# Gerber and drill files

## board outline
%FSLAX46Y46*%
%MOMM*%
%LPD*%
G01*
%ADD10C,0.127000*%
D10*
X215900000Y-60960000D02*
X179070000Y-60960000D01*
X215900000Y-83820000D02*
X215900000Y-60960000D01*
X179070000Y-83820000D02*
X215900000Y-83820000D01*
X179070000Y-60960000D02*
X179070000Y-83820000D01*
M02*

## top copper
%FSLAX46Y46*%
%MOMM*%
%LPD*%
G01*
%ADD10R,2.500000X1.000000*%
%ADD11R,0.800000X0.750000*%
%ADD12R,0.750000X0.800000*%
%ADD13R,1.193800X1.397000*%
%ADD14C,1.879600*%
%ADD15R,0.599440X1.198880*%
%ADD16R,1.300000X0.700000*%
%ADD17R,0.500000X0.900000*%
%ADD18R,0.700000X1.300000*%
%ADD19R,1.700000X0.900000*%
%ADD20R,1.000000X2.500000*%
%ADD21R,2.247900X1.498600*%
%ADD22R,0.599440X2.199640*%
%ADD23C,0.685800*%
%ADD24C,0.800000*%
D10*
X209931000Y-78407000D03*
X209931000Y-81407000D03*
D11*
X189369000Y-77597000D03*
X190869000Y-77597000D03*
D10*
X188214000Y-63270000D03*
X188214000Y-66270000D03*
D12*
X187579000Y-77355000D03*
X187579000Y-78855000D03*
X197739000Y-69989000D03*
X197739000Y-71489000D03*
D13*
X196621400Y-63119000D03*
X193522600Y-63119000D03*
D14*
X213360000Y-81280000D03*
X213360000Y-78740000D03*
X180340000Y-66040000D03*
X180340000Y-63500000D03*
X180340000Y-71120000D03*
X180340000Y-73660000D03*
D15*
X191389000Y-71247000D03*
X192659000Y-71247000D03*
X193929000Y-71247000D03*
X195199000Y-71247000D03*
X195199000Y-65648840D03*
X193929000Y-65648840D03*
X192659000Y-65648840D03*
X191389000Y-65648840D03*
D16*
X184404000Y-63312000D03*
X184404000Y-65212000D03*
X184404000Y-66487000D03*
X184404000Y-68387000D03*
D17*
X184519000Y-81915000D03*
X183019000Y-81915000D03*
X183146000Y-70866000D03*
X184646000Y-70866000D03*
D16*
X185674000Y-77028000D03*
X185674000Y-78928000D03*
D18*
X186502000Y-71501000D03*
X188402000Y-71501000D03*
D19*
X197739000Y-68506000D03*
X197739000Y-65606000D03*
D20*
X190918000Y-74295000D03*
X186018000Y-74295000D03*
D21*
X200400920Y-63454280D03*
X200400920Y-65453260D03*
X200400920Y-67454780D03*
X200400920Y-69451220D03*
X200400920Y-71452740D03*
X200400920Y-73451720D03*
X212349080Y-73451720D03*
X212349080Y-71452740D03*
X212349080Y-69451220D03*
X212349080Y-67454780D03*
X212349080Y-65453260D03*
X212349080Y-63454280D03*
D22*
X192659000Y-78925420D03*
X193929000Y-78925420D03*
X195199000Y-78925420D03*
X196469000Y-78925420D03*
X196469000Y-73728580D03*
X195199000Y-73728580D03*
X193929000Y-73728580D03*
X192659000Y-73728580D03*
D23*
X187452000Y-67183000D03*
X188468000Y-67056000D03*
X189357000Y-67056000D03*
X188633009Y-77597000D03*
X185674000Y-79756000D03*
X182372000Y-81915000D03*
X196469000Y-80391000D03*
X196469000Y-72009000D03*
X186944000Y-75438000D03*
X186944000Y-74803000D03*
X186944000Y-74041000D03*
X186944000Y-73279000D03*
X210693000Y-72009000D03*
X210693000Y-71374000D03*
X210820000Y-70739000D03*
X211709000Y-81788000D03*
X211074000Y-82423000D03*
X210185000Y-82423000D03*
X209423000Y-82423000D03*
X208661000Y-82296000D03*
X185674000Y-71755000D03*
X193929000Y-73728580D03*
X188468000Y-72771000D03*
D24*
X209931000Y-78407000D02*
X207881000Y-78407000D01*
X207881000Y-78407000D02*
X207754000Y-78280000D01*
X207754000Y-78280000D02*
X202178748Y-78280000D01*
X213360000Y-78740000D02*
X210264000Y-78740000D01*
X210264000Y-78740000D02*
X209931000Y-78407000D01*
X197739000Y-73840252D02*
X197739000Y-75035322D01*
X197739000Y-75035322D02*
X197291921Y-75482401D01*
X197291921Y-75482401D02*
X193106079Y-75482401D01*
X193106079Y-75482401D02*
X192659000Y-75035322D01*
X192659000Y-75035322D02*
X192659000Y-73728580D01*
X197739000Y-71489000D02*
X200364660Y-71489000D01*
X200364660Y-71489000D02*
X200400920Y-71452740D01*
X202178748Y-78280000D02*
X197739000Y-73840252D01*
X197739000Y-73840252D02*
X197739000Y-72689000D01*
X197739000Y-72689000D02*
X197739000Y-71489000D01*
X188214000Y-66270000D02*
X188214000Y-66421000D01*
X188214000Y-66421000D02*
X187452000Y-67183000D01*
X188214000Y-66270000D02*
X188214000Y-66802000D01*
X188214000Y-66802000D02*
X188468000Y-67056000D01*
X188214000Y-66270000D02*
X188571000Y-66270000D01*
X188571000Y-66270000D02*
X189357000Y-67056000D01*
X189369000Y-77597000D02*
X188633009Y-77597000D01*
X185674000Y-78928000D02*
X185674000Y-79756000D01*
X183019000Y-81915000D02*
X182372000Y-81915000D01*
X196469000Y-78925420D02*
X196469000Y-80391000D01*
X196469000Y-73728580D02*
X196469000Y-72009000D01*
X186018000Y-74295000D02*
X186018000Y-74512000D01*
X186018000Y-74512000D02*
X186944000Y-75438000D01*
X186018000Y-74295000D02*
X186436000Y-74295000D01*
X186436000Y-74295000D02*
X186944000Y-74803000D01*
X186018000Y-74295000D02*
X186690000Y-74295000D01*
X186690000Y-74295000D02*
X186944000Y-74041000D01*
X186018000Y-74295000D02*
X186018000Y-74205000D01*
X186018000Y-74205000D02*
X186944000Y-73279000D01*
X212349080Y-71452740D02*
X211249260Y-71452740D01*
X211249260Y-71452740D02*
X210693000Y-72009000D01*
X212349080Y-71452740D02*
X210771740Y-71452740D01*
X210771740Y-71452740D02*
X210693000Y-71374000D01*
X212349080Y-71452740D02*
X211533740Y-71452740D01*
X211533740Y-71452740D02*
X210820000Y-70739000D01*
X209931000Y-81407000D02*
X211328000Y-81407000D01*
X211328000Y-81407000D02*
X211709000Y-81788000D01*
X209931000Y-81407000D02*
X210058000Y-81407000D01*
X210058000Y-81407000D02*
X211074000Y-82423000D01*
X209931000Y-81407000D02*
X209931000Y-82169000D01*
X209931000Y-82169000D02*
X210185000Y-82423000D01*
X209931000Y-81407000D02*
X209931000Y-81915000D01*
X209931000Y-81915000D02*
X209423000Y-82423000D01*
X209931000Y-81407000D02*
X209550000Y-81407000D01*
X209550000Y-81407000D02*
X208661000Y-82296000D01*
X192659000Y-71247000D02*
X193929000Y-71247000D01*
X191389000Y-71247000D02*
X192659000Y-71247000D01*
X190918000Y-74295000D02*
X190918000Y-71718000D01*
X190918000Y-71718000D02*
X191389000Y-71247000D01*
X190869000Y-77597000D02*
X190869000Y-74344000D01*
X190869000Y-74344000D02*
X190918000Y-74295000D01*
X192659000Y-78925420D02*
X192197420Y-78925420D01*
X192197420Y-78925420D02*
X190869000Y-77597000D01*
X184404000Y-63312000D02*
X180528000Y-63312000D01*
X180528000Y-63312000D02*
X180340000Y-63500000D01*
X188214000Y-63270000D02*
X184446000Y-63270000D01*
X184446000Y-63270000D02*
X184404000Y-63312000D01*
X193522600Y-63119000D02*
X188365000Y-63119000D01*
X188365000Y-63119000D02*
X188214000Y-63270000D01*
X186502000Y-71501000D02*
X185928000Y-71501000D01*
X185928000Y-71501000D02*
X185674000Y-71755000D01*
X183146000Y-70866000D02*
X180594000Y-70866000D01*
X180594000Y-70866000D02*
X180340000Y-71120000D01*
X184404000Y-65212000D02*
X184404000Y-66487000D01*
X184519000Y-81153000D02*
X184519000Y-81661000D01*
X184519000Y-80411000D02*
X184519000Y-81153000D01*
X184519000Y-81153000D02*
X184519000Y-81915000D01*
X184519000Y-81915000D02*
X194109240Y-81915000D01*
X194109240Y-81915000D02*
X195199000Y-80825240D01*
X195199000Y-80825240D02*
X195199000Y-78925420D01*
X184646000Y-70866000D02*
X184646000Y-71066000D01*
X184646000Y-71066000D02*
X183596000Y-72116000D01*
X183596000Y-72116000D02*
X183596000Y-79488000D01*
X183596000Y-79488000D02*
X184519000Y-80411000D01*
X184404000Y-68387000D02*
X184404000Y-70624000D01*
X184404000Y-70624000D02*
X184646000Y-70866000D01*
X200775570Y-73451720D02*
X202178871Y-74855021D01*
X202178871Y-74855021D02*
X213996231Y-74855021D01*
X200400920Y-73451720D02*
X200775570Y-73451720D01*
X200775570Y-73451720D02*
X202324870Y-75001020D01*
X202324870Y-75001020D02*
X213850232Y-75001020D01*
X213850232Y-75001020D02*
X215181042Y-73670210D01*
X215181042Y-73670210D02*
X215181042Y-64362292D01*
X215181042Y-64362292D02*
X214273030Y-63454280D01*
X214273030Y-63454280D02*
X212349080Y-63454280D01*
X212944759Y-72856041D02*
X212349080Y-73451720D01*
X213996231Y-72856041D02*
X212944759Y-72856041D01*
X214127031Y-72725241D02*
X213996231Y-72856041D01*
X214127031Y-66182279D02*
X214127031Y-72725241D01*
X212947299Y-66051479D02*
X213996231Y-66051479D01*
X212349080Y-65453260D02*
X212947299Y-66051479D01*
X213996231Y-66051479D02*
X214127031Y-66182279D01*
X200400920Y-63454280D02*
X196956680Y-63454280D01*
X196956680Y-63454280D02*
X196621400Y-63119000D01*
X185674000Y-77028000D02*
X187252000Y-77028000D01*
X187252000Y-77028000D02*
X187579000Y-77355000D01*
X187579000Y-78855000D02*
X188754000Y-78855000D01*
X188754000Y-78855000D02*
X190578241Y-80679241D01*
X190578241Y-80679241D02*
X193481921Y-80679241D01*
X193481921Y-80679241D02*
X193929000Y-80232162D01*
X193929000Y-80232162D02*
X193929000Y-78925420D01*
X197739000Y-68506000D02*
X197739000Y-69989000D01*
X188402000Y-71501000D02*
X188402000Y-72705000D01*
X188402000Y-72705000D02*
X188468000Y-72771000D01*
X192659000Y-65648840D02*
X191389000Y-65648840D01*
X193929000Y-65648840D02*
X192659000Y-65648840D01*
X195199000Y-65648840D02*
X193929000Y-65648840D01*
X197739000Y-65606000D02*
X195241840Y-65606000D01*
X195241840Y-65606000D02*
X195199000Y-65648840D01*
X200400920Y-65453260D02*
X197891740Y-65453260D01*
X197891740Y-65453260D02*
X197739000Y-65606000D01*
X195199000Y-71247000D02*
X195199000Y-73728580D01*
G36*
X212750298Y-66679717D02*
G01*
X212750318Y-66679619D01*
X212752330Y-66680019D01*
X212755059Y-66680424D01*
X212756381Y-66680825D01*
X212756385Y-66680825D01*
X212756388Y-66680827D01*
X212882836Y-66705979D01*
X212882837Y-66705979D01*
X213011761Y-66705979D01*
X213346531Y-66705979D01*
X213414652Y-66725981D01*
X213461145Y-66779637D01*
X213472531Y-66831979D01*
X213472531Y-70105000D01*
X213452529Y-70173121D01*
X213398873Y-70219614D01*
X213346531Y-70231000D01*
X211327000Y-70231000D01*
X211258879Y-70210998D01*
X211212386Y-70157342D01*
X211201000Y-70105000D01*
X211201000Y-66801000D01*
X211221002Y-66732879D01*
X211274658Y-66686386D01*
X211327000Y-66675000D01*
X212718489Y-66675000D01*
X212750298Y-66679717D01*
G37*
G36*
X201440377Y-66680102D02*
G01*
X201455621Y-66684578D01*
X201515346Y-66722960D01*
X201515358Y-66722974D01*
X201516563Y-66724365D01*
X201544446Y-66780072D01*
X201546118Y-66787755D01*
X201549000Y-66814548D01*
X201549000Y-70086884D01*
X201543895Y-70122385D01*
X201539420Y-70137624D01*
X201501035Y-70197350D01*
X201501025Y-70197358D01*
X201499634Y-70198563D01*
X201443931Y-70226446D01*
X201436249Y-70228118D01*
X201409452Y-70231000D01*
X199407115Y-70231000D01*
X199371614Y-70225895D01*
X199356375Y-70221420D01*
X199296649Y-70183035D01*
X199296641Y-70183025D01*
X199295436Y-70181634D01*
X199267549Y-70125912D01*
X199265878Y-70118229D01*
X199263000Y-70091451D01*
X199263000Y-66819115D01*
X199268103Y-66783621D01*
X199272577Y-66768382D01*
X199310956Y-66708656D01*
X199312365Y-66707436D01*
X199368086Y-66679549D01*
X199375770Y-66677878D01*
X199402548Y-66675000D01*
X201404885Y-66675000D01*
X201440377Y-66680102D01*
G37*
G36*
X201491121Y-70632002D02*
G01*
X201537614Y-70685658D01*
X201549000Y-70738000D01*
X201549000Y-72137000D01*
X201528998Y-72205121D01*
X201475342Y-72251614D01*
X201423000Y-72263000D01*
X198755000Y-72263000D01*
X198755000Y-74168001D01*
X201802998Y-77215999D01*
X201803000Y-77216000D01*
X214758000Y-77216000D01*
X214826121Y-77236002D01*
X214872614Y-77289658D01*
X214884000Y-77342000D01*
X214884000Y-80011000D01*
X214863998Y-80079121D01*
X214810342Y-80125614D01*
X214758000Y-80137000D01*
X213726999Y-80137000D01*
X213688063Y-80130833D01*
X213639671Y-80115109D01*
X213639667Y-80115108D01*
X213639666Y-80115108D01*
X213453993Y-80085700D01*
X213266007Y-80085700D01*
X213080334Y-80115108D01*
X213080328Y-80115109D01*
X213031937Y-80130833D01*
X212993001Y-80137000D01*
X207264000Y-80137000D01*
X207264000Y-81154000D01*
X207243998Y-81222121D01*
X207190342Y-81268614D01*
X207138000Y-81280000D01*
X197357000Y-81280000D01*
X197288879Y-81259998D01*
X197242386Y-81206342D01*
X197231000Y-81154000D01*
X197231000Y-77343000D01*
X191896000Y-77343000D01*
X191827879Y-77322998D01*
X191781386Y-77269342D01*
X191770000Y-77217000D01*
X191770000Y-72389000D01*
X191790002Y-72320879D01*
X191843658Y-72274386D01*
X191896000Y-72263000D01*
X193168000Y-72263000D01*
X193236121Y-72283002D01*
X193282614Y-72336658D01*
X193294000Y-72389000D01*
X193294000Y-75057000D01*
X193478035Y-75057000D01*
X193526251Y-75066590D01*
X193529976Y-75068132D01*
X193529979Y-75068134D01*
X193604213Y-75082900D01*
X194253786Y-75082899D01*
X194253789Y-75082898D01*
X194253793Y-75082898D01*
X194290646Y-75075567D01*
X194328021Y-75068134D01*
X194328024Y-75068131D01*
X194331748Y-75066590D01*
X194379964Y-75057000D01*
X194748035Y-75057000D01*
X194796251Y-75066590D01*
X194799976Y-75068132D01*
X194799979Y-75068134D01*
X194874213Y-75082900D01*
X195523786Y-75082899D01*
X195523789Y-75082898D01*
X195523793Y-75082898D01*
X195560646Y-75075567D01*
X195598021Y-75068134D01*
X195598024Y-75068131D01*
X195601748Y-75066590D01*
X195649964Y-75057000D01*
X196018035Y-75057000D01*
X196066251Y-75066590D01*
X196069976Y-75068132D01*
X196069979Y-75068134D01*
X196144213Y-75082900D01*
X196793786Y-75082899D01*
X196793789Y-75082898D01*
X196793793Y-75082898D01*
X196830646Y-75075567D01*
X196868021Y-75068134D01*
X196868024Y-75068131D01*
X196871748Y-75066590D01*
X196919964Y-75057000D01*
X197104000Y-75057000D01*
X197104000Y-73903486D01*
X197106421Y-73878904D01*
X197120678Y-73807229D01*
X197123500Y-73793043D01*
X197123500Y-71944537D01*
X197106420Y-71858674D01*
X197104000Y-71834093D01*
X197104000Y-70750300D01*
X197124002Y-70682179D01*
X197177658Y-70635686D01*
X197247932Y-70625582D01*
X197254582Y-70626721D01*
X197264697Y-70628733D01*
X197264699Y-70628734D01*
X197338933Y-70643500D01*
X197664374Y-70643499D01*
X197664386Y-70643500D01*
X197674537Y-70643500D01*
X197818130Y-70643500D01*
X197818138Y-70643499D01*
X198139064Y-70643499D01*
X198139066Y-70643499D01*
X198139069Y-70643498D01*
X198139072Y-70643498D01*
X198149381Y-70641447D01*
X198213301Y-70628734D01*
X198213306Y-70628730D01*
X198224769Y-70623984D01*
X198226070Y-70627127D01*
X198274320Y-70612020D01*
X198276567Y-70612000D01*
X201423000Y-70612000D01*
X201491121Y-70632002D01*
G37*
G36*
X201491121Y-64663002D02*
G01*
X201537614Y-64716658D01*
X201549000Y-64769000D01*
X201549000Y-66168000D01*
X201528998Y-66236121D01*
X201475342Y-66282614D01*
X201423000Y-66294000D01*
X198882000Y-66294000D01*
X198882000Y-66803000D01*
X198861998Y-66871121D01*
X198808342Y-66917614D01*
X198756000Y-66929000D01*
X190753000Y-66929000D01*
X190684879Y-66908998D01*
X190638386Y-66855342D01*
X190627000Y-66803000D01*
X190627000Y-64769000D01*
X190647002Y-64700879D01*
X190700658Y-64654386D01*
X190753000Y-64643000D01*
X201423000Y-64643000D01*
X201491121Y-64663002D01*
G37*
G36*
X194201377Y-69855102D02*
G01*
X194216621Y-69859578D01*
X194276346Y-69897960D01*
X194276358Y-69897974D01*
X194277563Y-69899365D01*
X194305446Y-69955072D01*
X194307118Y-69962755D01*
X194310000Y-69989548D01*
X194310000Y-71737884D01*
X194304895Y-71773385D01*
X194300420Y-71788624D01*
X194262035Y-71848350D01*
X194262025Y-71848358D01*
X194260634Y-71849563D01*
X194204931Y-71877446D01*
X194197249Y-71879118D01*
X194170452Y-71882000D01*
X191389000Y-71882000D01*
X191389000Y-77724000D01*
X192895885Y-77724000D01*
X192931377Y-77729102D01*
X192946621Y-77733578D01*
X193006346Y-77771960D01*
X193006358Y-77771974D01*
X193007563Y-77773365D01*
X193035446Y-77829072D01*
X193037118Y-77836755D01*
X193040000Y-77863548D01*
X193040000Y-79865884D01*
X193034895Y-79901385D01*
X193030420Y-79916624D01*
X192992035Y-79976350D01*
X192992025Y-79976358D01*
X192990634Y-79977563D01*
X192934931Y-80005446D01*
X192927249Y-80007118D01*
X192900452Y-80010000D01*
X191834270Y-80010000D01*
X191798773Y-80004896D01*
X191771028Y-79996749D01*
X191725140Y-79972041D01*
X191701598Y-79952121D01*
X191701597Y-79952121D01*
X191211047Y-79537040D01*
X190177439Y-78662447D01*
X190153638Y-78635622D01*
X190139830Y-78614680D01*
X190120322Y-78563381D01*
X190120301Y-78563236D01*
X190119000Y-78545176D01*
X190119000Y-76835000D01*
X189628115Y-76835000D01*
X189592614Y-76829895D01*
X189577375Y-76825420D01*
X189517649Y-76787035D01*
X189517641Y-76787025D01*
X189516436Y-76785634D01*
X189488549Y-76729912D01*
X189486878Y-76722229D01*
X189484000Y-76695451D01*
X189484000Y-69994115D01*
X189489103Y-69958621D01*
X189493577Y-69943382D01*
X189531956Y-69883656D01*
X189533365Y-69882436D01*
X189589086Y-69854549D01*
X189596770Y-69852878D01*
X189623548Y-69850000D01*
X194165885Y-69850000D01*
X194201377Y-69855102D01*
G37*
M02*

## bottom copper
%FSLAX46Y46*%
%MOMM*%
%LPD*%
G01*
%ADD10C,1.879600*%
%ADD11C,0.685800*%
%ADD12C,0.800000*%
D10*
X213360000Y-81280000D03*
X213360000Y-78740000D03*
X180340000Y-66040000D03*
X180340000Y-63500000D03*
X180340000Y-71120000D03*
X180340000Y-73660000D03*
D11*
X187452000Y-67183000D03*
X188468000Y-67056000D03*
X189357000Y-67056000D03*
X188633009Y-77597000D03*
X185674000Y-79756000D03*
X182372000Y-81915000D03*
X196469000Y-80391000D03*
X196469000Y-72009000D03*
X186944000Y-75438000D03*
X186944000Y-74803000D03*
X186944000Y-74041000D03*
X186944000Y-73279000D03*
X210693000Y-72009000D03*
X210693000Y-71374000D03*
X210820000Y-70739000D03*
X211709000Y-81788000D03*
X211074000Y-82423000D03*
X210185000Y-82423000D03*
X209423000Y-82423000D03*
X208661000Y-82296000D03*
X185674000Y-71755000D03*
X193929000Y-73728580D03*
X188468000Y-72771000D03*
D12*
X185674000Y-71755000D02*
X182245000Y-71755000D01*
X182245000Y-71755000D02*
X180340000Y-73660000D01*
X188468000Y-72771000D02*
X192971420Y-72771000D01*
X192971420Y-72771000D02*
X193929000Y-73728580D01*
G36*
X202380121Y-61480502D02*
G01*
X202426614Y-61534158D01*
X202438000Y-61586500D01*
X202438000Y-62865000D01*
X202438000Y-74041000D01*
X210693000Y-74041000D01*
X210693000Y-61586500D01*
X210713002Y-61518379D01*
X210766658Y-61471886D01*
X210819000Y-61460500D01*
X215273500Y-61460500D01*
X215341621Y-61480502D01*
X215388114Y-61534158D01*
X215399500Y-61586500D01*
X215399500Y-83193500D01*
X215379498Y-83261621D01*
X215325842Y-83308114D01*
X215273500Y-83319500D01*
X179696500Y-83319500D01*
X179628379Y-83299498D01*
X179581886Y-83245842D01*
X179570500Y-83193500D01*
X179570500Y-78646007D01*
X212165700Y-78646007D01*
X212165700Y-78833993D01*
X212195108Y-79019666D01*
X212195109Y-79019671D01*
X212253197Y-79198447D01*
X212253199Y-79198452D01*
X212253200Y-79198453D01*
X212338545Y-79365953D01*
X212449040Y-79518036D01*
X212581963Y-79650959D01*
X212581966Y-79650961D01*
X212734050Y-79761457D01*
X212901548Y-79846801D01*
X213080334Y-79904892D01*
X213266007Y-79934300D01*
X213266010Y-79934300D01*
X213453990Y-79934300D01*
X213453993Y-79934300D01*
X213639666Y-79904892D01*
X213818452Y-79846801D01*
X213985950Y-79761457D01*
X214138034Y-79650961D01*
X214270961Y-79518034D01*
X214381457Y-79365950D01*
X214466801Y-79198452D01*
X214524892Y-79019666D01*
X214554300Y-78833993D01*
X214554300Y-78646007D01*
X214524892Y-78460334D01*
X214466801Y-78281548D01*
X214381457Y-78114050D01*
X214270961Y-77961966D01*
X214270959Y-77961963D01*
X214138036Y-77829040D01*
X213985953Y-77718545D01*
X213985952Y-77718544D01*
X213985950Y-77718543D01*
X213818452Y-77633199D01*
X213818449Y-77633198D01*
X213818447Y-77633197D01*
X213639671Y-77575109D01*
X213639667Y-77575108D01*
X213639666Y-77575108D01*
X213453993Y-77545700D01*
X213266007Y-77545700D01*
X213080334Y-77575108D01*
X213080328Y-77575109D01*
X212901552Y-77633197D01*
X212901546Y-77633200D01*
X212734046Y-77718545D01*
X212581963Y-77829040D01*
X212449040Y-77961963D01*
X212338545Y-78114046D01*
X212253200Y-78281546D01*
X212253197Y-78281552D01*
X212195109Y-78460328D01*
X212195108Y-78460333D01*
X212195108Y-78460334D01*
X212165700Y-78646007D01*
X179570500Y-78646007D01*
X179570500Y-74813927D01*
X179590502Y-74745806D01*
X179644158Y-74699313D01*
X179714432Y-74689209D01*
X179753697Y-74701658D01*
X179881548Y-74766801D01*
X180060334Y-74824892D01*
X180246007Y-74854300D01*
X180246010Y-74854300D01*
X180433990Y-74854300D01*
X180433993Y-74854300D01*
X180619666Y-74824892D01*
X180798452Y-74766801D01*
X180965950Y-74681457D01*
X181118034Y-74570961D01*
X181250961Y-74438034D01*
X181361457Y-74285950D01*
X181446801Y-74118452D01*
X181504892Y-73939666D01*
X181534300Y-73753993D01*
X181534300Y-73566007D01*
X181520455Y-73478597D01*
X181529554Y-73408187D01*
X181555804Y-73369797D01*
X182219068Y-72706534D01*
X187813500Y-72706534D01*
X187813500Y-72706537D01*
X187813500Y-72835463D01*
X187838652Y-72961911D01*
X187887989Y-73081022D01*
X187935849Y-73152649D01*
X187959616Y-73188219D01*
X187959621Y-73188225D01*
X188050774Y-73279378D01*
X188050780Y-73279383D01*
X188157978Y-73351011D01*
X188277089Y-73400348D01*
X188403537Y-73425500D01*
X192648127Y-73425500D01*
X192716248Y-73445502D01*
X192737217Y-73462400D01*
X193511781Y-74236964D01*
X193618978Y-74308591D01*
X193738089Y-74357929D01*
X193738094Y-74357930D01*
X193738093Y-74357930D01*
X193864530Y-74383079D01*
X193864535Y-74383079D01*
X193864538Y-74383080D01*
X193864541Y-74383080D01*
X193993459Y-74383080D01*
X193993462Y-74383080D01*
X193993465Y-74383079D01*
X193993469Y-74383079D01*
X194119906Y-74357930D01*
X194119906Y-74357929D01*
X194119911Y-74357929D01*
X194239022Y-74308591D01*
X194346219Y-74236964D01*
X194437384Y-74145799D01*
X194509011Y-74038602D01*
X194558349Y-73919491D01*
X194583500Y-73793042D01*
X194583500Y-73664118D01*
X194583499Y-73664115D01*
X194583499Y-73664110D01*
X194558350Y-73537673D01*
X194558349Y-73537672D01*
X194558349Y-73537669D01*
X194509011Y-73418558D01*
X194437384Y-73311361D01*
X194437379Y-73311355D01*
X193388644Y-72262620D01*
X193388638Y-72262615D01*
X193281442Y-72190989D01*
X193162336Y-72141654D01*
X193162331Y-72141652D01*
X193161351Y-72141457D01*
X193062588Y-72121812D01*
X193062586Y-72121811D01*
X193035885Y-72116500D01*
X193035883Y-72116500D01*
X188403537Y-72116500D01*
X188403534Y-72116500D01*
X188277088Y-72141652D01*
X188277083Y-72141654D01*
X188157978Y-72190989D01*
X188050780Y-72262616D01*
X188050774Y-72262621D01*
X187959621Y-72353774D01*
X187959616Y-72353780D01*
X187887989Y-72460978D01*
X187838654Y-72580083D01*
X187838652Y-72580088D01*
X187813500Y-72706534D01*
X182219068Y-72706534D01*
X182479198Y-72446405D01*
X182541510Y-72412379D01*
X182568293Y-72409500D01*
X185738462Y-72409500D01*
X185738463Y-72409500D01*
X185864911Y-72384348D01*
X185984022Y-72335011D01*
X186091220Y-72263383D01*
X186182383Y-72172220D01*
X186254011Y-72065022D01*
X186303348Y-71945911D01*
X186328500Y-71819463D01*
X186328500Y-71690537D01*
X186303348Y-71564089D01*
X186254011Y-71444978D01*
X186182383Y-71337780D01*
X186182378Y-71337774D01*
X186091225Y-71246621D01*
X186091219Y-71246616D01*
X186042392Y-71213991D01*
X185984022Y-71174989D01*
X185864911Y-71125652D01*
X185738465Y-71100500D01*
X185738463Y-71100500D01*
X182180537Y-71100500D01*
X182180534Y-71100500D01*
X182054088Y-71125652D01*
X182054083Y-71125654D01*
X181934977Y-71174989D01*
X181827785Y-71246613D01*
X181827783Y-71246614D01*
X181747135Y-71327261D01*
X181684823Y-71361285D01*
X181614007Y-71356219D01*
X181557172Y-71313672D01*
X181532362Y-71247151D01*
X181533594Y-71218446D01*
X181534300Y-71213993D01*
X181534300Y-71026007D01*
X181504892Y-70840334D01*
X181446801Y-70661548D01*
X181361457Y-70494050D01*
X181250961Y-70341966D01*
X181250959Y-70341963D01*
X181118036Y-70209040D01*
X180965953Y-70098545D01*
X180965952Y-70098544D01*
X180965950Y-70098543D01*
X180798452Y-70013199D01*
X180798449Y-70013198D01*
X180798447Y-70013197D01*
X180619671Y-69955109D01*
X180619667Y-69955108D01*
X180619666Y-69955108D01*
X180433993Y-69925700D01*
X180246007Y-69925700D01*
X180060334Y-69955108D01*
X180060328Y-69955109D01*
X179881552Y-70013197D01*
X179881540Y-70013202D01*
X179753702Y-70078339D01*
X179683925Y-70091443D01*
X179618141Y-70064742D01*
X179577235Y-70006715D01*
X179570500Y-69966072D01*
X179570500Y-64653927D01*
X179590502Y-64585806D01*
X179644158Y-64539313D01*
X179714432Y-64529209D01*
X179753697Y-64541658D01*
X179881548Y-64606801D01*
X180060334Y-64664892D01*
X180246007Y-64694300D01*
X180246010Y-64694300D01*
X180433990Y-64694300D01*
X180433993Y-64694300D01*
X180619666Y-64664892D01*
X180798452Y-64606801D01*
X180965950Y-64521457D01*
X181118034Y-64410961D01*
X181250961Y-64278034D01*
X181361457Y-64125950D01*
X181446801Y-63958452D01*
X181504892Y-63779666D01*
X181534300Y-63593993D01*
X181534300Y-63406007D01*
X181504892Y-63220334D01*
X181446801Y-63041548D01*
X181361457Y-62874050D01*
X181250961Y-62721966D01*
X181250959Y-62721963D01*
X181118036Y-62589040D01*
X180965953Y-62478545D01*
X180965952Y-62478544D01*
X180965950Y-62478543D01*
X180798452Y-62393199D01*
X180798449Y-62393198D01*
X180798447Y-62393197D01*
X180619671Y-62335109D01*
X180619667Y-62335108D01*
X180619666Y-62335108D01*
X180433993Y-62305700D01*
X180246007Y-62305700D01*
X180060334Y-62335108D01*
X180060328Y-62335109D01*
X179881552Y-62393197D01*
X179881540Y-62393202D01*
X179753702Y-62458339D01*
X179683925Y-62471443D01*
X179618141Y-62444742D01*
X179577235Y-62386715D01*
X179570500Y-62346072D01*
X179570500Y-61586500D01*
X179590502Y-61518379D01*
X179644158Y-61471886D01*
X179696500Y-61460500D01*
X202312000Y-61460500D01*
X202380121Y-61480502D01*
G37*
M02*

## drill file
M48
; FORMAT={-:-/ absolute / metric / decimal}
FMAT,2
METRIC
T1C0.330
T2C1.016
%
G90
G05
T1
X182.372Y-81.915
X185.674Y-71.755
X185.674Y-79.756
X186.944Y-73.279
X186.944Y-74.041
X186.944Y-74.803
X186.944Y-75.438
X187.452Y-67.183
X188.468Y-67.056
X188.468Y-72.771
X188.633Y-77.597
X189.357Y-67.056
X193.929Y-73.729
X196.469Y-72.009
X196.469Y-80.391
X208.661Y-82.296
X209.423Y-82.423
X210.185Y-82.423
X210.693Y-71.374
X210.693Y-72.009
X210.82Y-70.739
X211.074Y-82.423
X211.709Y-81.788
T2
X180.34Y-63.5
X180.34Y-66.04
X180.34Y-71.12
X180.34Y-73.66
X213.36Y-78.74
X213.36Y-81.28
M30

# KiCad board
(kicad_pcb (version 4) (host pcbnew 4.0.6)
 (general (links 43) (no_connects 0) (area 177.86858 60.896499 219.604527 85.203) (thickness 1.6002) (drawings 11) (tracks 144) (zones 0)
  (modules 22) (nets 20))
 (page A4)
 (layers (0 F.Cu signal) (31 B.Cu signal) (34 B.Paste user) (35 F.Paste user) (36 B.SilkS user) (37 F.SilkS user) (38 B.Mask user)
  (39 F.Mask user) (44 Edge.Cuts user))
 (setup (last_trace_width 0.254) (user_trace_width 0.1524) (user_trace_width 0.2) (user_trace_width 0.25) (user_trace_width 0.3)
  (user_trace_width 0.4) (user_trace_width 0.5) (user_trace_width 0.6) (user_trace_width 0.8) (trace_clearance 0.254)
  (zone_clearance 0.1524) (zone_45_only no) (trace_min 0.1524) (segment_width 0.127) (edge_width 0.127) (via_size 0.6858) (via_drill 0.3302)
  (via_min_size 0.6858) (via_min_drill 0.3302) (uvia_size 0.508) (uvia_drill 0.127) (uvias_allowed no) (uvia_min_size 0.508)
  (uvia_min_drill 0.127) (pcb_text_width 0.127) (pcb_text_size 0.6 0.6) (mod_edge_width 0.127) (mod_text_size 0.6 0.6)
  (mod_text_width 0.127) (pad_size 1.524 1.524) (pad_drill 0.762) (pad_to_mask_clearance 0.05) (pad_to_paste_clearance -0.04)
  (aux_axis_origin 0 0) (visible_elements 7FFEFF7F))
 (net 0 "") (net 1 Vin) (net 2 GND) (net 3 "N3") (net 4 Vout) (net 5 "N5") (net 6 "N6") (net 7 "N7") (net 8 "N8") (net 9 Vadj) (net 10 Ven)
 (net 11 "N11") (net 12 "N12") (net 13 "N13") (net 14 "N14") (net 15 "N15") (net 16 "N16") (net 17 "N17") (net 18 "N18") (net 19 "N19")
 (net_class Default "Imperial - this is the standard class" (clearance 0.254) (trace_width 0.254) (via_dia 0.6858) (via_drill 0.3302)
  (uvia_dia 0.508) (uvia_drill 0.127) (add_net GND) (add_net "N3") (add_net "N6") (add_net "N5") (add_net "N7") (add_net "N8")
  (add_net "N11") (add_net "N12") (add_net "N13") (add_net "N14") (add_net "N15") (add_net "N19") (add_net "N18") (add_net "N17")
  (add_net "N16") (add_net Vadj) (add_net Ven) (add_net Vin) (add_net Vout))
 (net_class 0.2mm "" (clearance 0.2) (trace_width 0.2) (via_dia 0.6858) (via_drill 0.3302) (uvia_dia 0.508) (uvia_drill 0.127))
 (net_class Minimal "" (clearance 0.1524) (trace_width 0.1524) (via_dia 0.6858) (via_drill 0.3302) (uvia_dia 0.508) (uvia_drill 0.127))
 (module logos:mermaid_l (layer B.Cu) (at 205.867 79.629 180)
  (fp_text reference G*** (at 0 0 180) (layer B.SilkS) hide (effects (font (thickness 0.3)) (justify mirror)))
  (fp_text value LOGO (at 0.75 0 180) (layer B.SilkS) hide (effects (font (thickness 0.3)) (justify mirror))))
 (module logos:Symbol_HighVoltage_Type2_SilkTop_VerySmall (layer F.Cu) (at 201.422 79.502)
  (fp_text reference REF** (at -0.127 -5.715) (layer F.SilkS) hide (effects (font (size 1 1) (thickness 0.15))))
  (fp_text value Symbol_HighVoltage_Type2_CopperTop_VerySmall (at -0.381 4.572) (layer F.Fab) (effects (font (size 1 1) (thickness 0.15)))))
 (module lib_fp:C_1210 (layer F.Cu) (at 209.931 79.907 270)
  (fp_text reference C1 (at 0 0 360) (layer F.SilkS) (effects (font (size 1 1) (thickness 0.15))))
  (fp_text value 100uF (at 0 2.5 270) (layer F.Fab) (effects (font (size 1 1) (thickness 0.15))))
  (pad 1 smd rect (at -1.5 0 270) (size 1 2.5) (layers F.Cu F.Paste F.Mask) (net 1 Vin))
  (pad 2 smd rect (at 1.5 0 270) (size 1 2.5) (layers F.Cu F.Paste F.Mask) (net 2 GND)))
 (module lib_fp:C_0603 (layer F.Cu) (at 190.119 77.597 180)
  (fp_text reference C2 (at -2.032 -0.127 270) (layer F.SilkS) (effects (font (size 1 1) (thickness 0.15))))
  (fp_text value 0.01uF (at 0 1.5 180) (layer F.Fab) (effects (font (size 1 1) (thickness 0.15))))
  (pad 2 smd rect (at 0.75 0 180) (size 0.8 0.75) (layers F.Cu F.Paste F.Mask) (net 2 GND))
  (pad 1 smd rect (at -0.75 0 180) (size 0.8 0.75) (layers F.Cu F.Paste F.Mask) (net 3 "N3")))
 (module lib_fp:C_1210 (layer F.Cu) (at 188.214 64.77 270)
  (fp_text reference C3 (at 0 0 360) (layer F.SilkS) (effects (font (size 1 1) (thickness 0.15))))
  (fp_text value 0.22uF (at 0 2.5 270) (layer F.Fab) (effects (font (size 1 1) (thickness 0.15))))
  (pad 1 smd rect (at -1.5 0 270) (size 1 2.5) (layers F.Cu F.Paste F.Mask) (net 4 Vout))
  (pad 2 smd rect (at 1.5 0 270) (size 1 2.5) (layers F.Cu F.Paste F.Mask) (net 2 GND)))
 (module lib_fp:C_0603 (layer F.Cu) (at 187.579 78.105 90)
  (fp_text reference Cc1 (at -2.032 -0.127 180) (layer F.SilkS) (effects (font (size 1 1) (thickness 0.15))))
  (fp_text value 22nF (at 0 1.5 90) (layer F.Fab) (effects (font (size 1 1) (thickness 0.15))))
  (pad 2 smd rect (at 0.75 0 90) (size 0.8 0.75) (layers F.Cu F.Paste F.Mask) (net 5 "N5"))
  (pad 1 smd rect (at -0.75 0 90) (size 0.8 0.75) (layers F.Cu F.Paste F.Mask) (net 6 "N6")))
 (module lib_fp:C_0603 (layer F.Cu) (at 197.739 70.739 90)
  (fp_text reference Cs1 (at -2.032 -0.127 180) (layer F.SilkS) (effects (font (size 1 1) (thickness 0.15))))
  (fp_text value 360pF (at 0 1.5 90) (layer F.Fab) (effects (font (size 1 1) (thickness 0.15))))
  (pad 2 smd rect (at 0.75 0 90) (size 0.8 0.75) (layers F.Cu F.Paste F.Mask) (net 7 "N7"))
  (pad 1 smd rect (at -0.75 0 90) (size 0.8 0.75) (layers F.Cu F.Paste F.Mask) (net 1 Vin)))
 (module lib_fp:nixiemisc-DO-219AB (layer F.Cu) (at 195.072 63.119)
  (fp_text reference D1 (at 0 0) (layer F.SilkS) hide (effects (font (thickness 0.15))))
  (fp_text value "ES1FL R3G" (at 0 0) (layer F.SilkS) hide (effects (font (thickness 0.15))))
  (pad A smd rect (at 1.5494 0 180) (size 1.1938 1.397) (layers F.Cu F.Paste F.Mask) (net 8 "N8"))
  (pad C smd rect (at -1.5494 0) (size 1.1938 1.397) (layers F.Cu F.Paste F.Mask) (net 4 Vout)))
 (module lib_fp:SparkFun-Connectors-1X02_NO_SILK (layer F.Cu) (at 213.36 81.28 90)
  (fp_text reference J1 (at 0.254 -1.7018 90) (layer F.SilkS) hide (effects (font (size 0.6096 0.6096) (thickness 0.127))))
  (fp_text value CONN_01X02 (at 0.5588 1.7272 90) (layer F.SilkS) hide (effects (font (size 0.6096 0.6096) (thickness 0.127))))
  (pad 1 thru_hole circle (at 0 0 90) (size 1.8796 1.8796) (drill 1.016) (layers *.Cu *.Paste *.Mask) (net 2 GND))
  (pad 2 thru_hole circle (at 2.54 0 90) (size 1.8796 1.8796) (drill 1.016) (layers *.Cu *.Paste *.Mask) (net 1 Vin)))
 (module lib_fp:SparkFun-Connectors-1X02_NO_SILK (layer F.Cu) (at 180.34 66.04 90)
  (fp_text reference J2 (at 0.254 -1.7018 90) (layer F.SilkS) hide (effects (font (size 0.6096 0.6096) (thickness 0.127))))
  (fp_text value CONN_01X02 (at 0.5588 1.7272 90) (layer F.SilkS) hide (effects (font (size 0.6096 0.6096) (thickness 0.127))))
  (pad 1 thru_hole circle (at 0 0 90) (size 1.8796 1.8796) (drill 1.016) (layers *.Cu *.Paste *.Mask) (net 2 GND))
  (pad 2 thru_hole circle (at 2.54 0 90) (size 1.8796 1.8796) (drill 1.016) (layers *.Cu *.Paste *.Mask) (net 4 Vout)))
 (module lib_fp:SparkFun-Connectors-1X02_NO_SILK (layer F.Cu) (at 180.34 71.12 270)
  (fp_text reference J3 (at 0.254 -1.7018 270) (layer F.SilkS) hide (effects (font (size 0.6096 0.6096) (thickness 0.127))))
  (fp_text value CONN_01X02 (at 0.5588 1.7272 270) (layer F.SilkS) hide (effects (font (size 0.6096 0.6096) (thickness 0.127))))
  (pad 1 thru_hole circle (at 0 0 270) (size 1.8796 1.8796) (drill 1.016) (layers *.Cu *.Paste *.Mask) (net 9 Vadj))
  (pad 2 thru_hole circle (at 2.54 0 270) (size 1.8796 1.8796) (drill 1.016) (layers *.Cu *.Paste *.Mask) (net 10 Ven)))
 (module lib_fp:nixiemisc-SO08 (layer F.Cu) (at 193.294 68.44792)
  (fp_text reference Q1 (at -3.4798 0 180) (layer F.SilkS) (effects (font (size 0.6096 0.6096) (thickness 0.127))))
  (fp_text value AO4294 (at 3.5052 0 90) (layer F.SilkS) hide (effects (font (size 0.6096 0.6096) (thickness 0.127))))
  (pad 1 smd rect (at -1.905 2.79908) (size 0.59944 1.19888) (layers F.Cu F.Paste F.Mask) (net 3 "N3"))
  (pad 2 smd rect (at -0.635 2.79908) (size 0.59944 1.19888) (layers F.Cu F.Paste F.Mask) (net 3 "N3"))
  (pad 3 smd rect (at 0.635 2.79908) (size 0.59944 1.19888) (layers F.Cu F.Paste F.Mask) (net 3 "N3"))
  (pad 4 smd rect (at 1.905 2.79908) (size 0.59944 1.19888) (layers F.Cu F.Paste F.Mask) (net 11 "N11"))
  (pad 5 smd rect (at 1.905 -2.79908) (size 0.59944 1.19888) (layers F.Cu F.Paste F.Mask) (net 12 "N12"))
  (pad 6 smd rect (at 0.635 -2.79908) (size 0.59944 1.19888) (layers F.Cu F.Paste F.Mask) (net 12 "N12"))
  (pad 7 smd rect (at -0.635 -2.79908) (size 0.59944 1.19888) (layers F.Cu F.Paste F.Mask) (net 12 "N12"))
  (pad 8 smd rect (at -1.905 -2.79908) (size 0.59944 1.19888) (layers F.Cu F.Paste F.Mask) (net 12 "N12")))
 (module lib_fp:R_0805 (layer F.Cu) (at 184.404 64.262 270)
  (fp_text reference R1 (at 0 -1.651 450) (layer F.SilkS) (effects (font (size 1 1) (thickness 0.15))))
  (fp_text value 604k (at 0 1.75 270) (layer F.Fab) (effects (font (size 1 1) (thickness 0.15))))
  (pad 1 smd rect (at -0.95 0 270) (size 0.7 1.3) (layers F.Cu F.Paste F.Mask) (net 4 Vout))
  (pad 2 smd rect (at 0.95 0 270) (size 0.7 1.3) (layers F.Cu F.Paste F.Mask) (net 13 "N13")))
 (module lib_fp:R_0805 (layer F.Cu) (at 184.404 67.437 270)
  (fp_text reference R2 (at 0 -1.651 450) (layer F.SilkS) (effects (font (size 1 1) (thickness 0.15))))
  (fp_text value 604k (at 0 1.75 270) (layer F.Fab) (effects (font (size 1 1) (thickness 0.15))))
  (pad 1 smd rect (at -0.95 0 270) (size 0.7 1.3) (layers F.Cu F.Paste F.Mask) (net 13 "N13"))
  (pad 2 smd rect (at 0.95 0 270) (size 0.7 1.3) (layers F.Cu F.Paste F.Mask) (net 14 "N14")))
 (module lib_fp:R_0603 (layer F.Cu) (at 183.769 81.915 180)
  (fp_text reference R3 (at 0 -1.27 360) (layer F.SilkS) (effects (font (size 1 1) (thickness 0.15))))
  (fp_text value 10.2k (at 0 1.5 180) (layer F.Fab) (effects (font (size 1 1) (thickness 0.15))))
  (pad 1 smd rect (at -0.75 0 180) (size 0.5 0.9) (layers F.Cu F.Paste F.Mask) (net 14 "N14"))
  (pad 2 smd rect (at 0.75 0 180) (size 0.5 0.9) (layers F.Cu F.Paste F.Mask) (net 2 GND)))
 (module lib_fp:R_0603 (layer F.Cu) (at 183.896 70.866)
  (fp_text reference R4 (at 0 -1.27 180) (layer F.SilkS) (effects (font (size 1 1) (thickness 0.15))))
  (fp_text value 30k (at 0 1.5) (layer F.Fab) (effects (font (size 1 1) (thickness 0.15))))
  (pad 1 smd rect (at -0.75 0) (size 0.5 0.9) (layers F.Cu F.Paste F.Mask) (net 9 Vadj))
  (pad 2 smd rect (at 0.75 0) (size 0.5 0.9) (layers F.Cu F.Paste F.Mask) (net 14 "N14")))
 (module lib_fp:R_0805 (layer F.Cu) (at 185.674 77.978 270)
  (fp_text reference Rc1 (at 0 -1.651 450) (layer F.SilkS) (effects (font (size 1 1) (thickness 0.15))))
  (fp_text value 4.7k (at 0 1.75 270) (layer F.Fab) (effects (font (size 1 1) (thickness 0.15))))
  (pad 1 smd rect (at -0.95 0 270) (size 0.7 1.3) (layers F.Cu F.Paste F.Mask) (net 5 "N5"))
  (pad 2 smd rect (at 0.95 0 270) (size 0.7 1.3) (layers F.Cu F.Paste F.Mask) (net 2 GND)))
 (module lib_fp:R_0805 (layer F.Cu) (at 187.452 71.501)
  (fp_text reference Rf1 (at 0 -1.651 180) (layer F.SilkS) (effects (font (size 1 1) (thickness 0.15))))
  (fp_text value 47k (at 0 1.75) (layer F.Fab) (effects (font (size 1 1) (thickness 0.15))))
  (pad 1 smd rect (at -0.95 0) (size 0.7 1.3) (layers F.Cu F.Paste F.Mask) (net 10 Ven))
  (pad 2 smd rect (at 0.95 0) (size 0.7 1.3) (layers F.Cu F.Paste F.Mask) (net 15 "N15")))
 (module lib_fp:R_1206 (layer F.Cu) (at 197.739 67.056 90)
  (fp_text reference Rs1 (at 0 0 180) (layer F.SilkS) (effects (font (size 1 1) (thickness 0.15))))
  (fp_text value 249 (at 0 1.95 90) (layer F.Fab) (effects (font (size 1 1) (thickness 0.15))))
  (pad 1 smd rect (at -1.45 0 90) (size 0.9 1.7) (layers F.Cu F.Paste F.Mask) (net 7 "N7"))
  (pad 2 smd rect (at 1.45 0 90) (size 0.9 1.7) (layers F.Cu F.Paste F.Mask) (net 12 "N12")))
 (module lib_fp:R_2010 (layer F.Cu) (at 188.468 74.295 180)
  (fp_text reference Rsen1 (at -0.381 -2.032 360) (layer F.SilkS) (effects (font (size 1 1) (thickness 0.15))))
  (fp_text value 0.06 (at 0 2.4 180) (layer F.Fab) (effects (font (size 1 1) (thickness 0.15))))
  (pad 1 smd rect (at -2.45 0 180) (size 1 2.5) (layers F.Cu F.Paste F.Mask) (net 3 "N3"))
  (pad 2 smd rect (at 2.45 0 180) (size 1 2.5) (layers F.Cu F.Paste F.Mask) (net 2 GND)))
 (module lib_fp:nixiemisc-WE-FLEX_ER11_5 (layer F.Cu) (at 206.375 68.453 90)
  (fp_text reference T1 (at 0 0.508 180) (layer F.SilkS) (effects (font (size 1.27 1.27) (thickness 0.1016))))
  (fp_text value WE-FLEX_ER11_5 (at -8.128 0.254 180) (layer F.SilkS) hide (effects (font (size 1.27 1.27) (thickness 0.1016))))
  (pad 1 smd rect (at 4.99872 -5.97408 270) (size 1.4986 2.2479) (layers F.Cu F.Paste F.Mask) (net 8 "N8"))
  (pad 2 smd rect (at 2.99974 -5.97408 270) (size 1.4986 2.2479) (layers F.Cu F.Paste F.Mask) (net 12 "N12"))
  (pad 3 smd rect (at 0.99822 -5.97408 270) (size 1.4986 2.2479) (layers F.Cu F.Paste F.Mask) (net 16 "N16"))
  (pad 4 smd rect (at -0.99822 -5.97408 270) (size 1.4986 2.2479) (layers F.Cu F.Paste F.Mask) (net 16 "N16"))
  (pad 5 smd rect (at -2.99974 -5.97408 270) (size 1.4986 2.2479) (layers F.Cu F.Paste F.Mask) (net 1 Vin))
  (pad 6 smd rect (at -4.99872 -5.97408 270) (size 1.4986 2.2479) (layers F.Cu F.Paste F.Mask) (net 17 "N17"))
  (pad 7 smd rect (at -4.99872 5.97408 270) (size 1.4986 2.2479) (layers F.Cu F.Paste F.Mask) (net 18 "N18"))
  (pad 8 smd rect (at -2.99974 5.97408 270) (size 1.4986 2.2479) (layers F.Cu F.Paste F.Mask) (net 2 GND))
  (pad 9 smd rect (at -0.99822 5.97408 270) (size 1.4986 2.2479) (layers F.Cu F.Paste F.Mask) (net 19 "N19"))
  (pad 10 smd rect (at 0.99822 5.97408 270) (size 1.4986 2.2479) (layers F.Cu F.Paste F.Mask) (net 19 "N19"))
  (pad 11 smd rect (at 2.99974 5.97408 270) (size 1.4986 2.2479) (layers F.Cu F.Paste F.Mask) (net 18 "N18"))
  (pad 12 smd rect (at 4.99872 5.97408 270) (size 1.4986 2.2479) (layers F.Cu F.Paste F.Mask) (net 17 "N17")))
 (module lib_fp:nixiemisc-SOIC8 (layer F.Cu) (at 194.564 76.327)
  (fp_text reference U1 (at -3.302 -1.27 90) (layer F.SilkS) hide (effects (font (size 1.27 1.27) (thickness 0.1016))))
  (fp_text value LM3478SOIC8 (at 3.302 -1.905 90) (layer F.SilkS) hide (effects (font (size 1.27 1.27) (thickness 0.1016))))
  (pad 1 smd rect (at -1.905 2.59842) (size 0.59944 2.19964) (layers F.Cu F.Paste F.Mask) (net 3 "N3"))
  (pad 2 smd rect (at -0.635 2.59842) (size 0.59944 2.19964) (layers F.Cu F.Paste F.Mask) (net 6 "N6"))
  (pad 3 smd rect (at 0.635 2.59842) (size 0.59944 2.19964) (layers F.Cu F.Paste F.Mask) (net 14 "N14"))
  (pad 4 smd rect (at 1.905 2.59842) (size 0.59944 2.19964) (layers F.Cu F.Paste F.Mask) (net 2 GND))
  (pad 5 smd rect (at 1.905 -2.59842) (size 0.59944 2.19964) (layers F.Cu F.Paste F.Mask) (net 2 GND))
  (pad 6 smd rect (at 0.635 -2.59842) (size 0.59944 2.19964) (layers F.Cu F.Paste F.Mask) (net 11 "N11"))
  (pad 7 smd rect (at -0.635 -2.59842) (size 0.59944 2.19964) (layers F.Cu F.Paste F.Mask) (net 15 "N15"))
  (pad 8 smd rect (at -1.905 -2.59842) (size 0.59944 2.19964) (layers F.Cu F.Paste F.Mask) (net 1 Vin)))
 (gr_line (start 215.9 60.96) (end 179.07 60.96) (layer Edge.Cuts) (width 0.127))
 (gr_line (start 215.9 83.82) (end 215.9 60.96) (layer Edge.Cuts) (width 0.127))
 (gr_line (start 179.07 83.82) (end 215.9 83.82) (layer Edge.Cuts) (width 0.127))
 (gr_line (start 179.07 60.96) (end 179.07 83.82) (layer Edge.Cuts) (width 0.127))
 (segment (start 209.931 78.407) (end 207.881 78.407) (width 0.8) (layer F.Cu) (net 1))
 (segment (start 207.881 78.407) (end 207.754 78.28) (width 0.8) (layer F.Cu) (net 1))
 (segment (start 207.754 78.28) (end 202.178748 78.28) (width 0.8) (layer F.Cu) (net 1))
 (segment (start 213.36 78.74) (end 210.264 78.74) (width 0.8) (layer F.Cu) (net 1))
 (segment (start 210.264 78.74) (end 209.931 78.407) (width 0.8) (layer F.Cu) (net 1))
 (segment (start 197.739 73.840252) (end 197.739 75.035322) (width 0.8) (layer F.Cu) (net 1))
 (segment (start 197.739 75.035322) (end 197.291921 75.482401) (width 0.8) (layer F.Cu) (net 1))
 (segment (start 197.291921 75.482401) (end 193.106079 75.482401) (width 0.8) (layer F.Cu) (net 1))
 (segment (start 193.106079 75.482401) (end 192.659 75.035322) (width 0.8) (layer F.Cu) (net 1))
 (segment (start 192.659 75.035322) (end 192.659 73.72858) (width 0.8) (layer F.Cu) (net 1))
 (segment (start 197.739 71.489) (end 200.36466 71.489) (width 0.8) (layer F.Cu) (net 1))
 (segment (start 200.36466 71.489) (end 200.40092 71.45274) (width 0.8) (layer F.Cu) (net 1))
 (segment (start 202.178748 78.28) (end 197.739 73.840252) (width 0.8) (layer F.Cu) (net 1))
 (segment (start 197.739 73.840252) (end 197.739 72.689) (width 0.8) (layer F.Cu) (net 1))
 (segment (start 197.739 72.689) (end 197.739 71.489) (width 0.8) (layer F.Cu) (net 1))
 (segment (start 188.214 66.27) (end 188.214 66.421) (width 0.8) (layer F.Cu) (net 2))
 (segment (start 188.214 66.421) (end 187.452 67.183) (width 0.8) (layer F.Cu) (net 2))
 (via (at 187.452 67.183) (size 0.6858) (drill 0.3302) (layers F.Cu B.Cu) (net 2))
 (segment (start 188.214 66.27) (end 188.214 66.802) (width 0.8) (layer F.Cu) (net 2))
 (segment (start 188.214 66.802) (end 188.468 67.056) (width 0.8) (layer F.Cu) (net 2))
 (via (at 188.468 67.056) (size 0.6858) (drill 0.3302) (layers F.Cu B.Cu) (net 2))
 (segment (start 188.214 66.27) (end 188.571 66.27) (width 0.8) (layer F.Cu) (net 2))
 (segment (start 188.571 66.27) (end 189.357 67.056) (width 0.8) (layer F.Cu) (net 2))
 (via (at 189.357 67.056) (size 0.6858) (drill 0.3302) (layers F.Cu B.Cu) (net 2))
 (segment (start 189.369 77.597) (end 188.633009 77.597) (width 0.8) (layer F.Cu) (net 2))
 (via (at 188.633009 77.597) (size 0.6858) (drill 0.3302) (layers F.Cu B.Cu) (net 2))
 (segment (start 185.674 78.928) (end 185.674 79.756) (width 0.8) (layer F.Cu) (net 2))
 (via (at 185.674 79.756) (size 0.6858) (drill 0.3302) (layers F.Cu B.Cu) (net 2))
 (segment (start 183.019 81.915) (end 182.372 81.915) (width 0.8) (layer F.Cu) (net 2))
 (via (at 182.372 81.915) (size 0.6858) (drill 0.3302) (layers F.Cu B.Cu) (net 2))
 (segment (start 196.469 78.92542) (end 196.469 80.391) (width 0.8) (layer F.Cu) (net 2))
 (via (at 196.469 80.391) (size 0.6858) (drill 0.3302) (layers F.Cu B.Cu) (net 2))
 (segment (start 196.469 73.72858) (end 196.469 72.009) (width 0.8) (layer F.Cu) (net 2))
 (via (at 196.469 72.009) (size 0.6858) (drill 0.3302) (layers F.Cu B.Cu) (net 2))
 (segment (start 186.018 74.295) (end 186.018 74.512) (width 0.8) (layer F.Cu) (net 2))
 (segment (start 186.018 74.512) (end 186.944 75.438) (width 0.8) (layer F.Cu) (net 2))
 (via (at 186.944 75.438) (size 0.6858) (drill 0.3302) (layers F.Cu B.Cu) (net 2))
 (segment (start 186.018 74.295) (end 186.436 74.295) (width 0.8) (layer F.Cu) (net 2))
 (segment (start 186.436 74.295) (end 186.944 74.803) (width 0.8) (layer F.Cu) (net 2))
 (via (at 186.944 74.803) (size 0.6858) (drill 0.3302) (layers F.Cu B.Cu) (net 2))
 (segment (start 186.018 74.295) (end 186.69 74.295) (width 0.8) (layer F.Cu) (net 2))
 (segment (start 186.69 74.295) (end 186.944 74.041) (width 0.8) (layer F.Cu) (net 2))
 (via (at 186.944 74.041) (size 0.6858) (drill 0.3302) (layers F.Cu B.Cu) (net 2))
 (segment (start 186.018 74.295) (end 186.018 74.205) (width 0.8) (layer F.Cu) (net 2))
 (segment (start 186.018 74.205) (end 186.944 73.279) (width 0.8) (layer F.Cu) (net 2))
 (via (at 186.944 73.279) (size 0.6858) (drill 0.3302) (layers F.Cu B.Cu) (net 2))
 (segment (start 212.34908 71.45274) (end 211.24926 71.45274) (width 0.8) (layer F.Cu) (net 2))
 (via (at 210.693 72.009) (size 0.6858) (drill 0.3302) (layers F.Cu B.Cu) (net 2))
 (segment (start 211.24926 71.45274) (end 210.693 72.009) (width 0.8) (layer F.Cu) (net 2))
 (segment (start 212.34908 71.45274) (end 210.77174 71.45274) (width 0.8) (layer F.Cu) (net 2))
 (segment (start 210.77174 71.45274) (end 210.693 71.374) (width 0.8) (layer F.Cu) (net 2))
 (via (at 210.693 71.374) (size 0.6858) (drill 0.3302) (layers F.Cu B.Cu) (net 2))
 (segment (start 212.34908 71.45274) (end 211.53374 71.45274) (width 0.8) (layer F.Cu) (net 2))
 (segment (start 211.53374 71.45274) (end 210.82 70.739) (width 0.8) (layer F.Cu) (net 2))
 (via (at 210.82 70.739) (size 0.6858) (drill 0.3302) (layers F.Cu B.Cu) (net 2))
 (segment (start 209.931 81.407) (end 211.328 81.407) (width 0.8) (layer F.Cu) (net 2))
 (segment (start 211.328 81.407) (end 211.709 81.788) (width 0.8) (layer F.Cu) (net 2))
 (via (at 211.709 81.788) (size 0.6858) (drill 0.3302) (layers F.Cu B.Cu) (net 2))
 (segment (start 209.931 81.407) (end 210.058 81.407) (width 0.8) (layer F.Cu) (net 2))
 (segment (start 210.058 81.407) (end 211.074 82.423) (width 0.8) (layer F.Cu) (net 2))
 (via (at 211.074 82.423) (size 0.6858) (drill 0.3302) (layers F.Cu B.Cu) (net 2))
 (segment (start 209.931 81.407) (end 209.931 82.169) (width 0.8) (layer F.Cu) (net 2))
 (segment (start 209.931 82.169) (end 210.185 82.423) (width 0.8) (layer F.Cu) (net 2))
 (via (at 210.185 82.423) (size 0.6858) (drill 0.3302) (layers F.Cu B.Cu) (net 2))
 (segment (start 209.931 81.407) (end 209.931 81.915) (width 0.8) (layer F.Cu) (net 2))
 (segment (start 209.931 81.915) (end 209.423 82.423) (width 0.8) (layer F.Cu) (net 2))
 (via (at 209.423 82.423) (size 0.6858) (drill 0.3302) (layers F.Cu B.Cu) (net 2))
 (segment (start 209.931 81.407) (end 209.55 81.407) (width 0.8) (layer F.Cu) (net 2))
 (segment (start 209.55 81.407) (end 208.661 82.296) (width 0.8) (layer F.Cu) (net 2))
 (via (at 208.661 82.296) (size 0.6858) (drill 0.3302) (layers F.Cu B.Cu) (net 2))
 (segment (start 192.659 71.247) (end 193.929 71.247) (width 0.8) (layer F.Cu) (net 3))
 (segment (start 191.389 71.247) (end 192.659 71.247) (width 0.8) (layer F.Cu) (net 3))
 (segment (start 190.918 74.295) (end 190.918 71.718) (width 0.8) (layer F.Cu) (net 3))
 (segment (start 190.918 71.718) (end 191.389 71.247) (width 0.8) (layer F.Cu) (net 3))
 (segment (start 190.869 77.597) (end 190.869 74.344) (width 0.8) (layer F.Cu) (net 3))
 (segment (start 190.869 74.344) (end 190.918 74.295) (width 0.8) (layer F.Cu) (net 3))
 (segment (start 192.659 78.92542) (end 192.19742 78.92542) (width 0.8) (layer F.Cu) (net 3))
 (segment (start 192.19742 78.92542) (end 190.869 77.597) (width 0.8) (layer F.Cu) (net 3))
 (segment (start 184.404 63.312) (end 180.528 63.312) (width 0.8) (layer F.Cu) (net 4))
 (segment (start 180.528 63.312) (end 180.34 63.5) (width 0.8) (layer F.Cu) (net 4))
 (segment (start 188.214 63.27) (end 184.446 63.27) (width 0.8) (layer F.Cu) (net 4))
 (segment (start 184.446 63.27) (end 184.404 63.312) (width 0.8) (layer F.Cu) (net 4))
 (segment (start 193.5226 63.119) (end 188.365 63.119) (width 0.8) (layer F.Cu) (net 4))
 (segment (start 188.365 63.119) (end 188.214 63.27) (width 0.8) (layer F.Cu) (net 4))
 (segment (start 185.674 71.755) (end 182.245 71.755) (width 0.8) (layer B.Cu) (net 10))
 (segment (start 182.245 71.755) (end 180.34 73.66) (width 0.8) (layer B.Cu) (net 10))
 (segment (start 186.502 71.501) (end 185.928 71.501) (width 0.8) (layer F.Cu) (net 10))
 (segment (start 185.928 71.501) (end 185.674 71.755) (width 0.8) (layer F.Cu) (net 10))
 (via (at 185.674 71.755) (size 0.6858) (drill 0.3302) (layers F.Cu B.Cu) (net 10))
 (segment (start 183.146 70.866) (end 180.594 70.866) (width 0.8) (layer F.Cu) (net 9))
 (segment (start 180.594 70.866) (end 180.34 71.12) (width 0.8) (layer F.Cu) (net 9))
 (segment (start 184.404 65.212) (end 184.404 66.487) (width 0.8) (layer F.Cu) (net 13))
 (segment (start 184.519 81.153) (end 184.519 81.661) (width 0.8) (layer F.Cu) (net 14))
 (segment (start 184.519 80.411) (end 184.519 81.153) (width 0.8) (layer F.Cu) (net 14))
 (segment (start 184.519 81.153) (end 184.519 81.915) (width 0.8) (layer F.Cu) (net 14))
 (segment (start 184.519 81.915) (end 194.10924 81.915) (width 0.8) (layer F.Cu) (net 14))
 (segment (start 194.10924 81.915) (end 195.199 80.82524) (width 0.8) (layer F.Cu) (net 14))
 (segment (start 195.199 80.82524) (end 195.199 78.92542) (width 0.8) (layer F.Cu) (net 14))
 (segment (start 184.646 70.866) (end 184.646 71.066) (width 0.8) (layer F.Cu) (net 14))
 (segment (start 184.646 71.066) (end 183.596 72.116) (width 0.8) (layer F.Cu) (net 14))
 (segment (start 183.596 72.116) (end 183.596 79.488) (width 0.8) (layer F.Cu) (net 14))
 (segment (start 183.596 79.488) (end 184.519 80.411) (width 0.8) (layer F.Cu) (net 14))
 (segment (start 184.404 68.387) (end 184.404 70.624) (width 0.8) (layer F.Cu) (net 14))
 (segment (start 184.404 70.624) (end 184.646 70.866) (width 0.8) (layer F.Cu) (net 14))
 (segment (start 200.77557 73.45172) (end 202.178871 74.855021) (width 0.8) (layer F.Cu) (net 17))
 (segment (start 202.178871 74.855021) (end 213.996231 74.855021) (width 0.8) (layer F.Cu) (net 17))
 (segment (start 200.40092 73.45172) (end 200.77557 73.45172) (width 0.8) (layer F.Cu) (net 17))
 (segment (start 200.77557 73.45172) (end 202.32487 75.00102) (width 0.8) (layer F.Cu) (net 17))
 (segment (start 202.32487 75.00102) (end 213.850232 75.00102) (width 0.8) (layer F.Cu) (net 17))
 (segment (start 213.850232 75.00102) (end 215.181042 73.67021) (width 0.8) (layer F.Cu) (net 17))
 (segment (start 215.181042 73.67021) (end 215.181042 64.362292) (width 0.8) (layer F.Cu) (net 17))
 (segment (start 215.181042 64.362292) (end 214.27303 63.45428) (width 0.8) (layer F.Cu) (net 17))
 (segment (start 214.27303 63.45428) (end 212.34908 63.45428) (width 0.8) (layer F.Cu) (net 17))
 (segment (start 212.944759 72.856041) (end 212.34908 73.45172) (width 0.8) (layer F.Cu) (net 18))
 (segment (start 213.996231 72.856041) (end 212.944759 72.856041) (width 0.8) (layer F.Cu) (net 18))
 (segment (start 214.127031 72.725241) (end 213.996231 72.856041) (width 0.8) (layer F.Cu) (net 18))
 (segment (start 214.127031 66.182279) (end 214.127031 72.725241) (width 0.8) (layer F.Cu) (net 18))
 (segment (start 212.947299 66.051479) (end 213.996231 66.051479) (width 0.8) (layer F.Cu) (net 18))
 (segment (start 212.34908 65.45326) (end 212.947299 66.051479) (width 0.8) (layer F.Cu) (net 18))
 (segment (start 213.996231 66.051479) (end 214.127031 66.182279) (width 0.8) (layer F.Cu) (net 18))
 (segment (start 200.40092 63.45428) (end 196.95668 63.45428) (width 0.8) (layer F.Cu) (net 8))
 (segment (start 196.95668 63.45428) (end 196.6214 63.119) (width 0.8) (layer F.Cu) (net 8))
 (segment (start 185.674 77.028) (end 187.252 77.028) (width 0.8) (layer F.Cu) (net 5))
 (segment (start 187.252 77.028) (end 187.579 77.355) (width 0.8) (layer F.Cu) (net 5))
 (segment (start 187.579 78.855) (end 188.754 78.855) (width 0.8) (layer F.Cu) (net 6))
 (segment (start 188.754 78.855) (end 190.578241 80.679241) (width 0.8) (layer F.Cu) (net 6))
 (segment (start 190.578241 80.679241) (end 193.481921 80.679241) (width 0.8) (layer F.Cu) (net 6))
 (segment (start 193.481921 80.679241) (end 193.929 80.232162) (width 0.8) (layer F.Cu) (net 6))
 (segment (start 193.929 80.232162) (end 193.929 78.92542) (width 0.8) (layer F.Cu) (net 6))
 (segment (start 197.739 68.506) (end 197.739 69.989) (width 0.8) (layer F.Cu) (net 7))
 (segment (start 188.468 72.771) (end 192.97142 72.771) (width 0.8) (layer B.Cu) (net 15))
 (segment (start 192.97142 72.771) (end 193.929 73.72858) (width 0.8) (layer B.Cu) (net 15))
 (via (at 193.929 73.72858) (size 0.6858) (drill 0.3302) (layers F.Cu B.Cu) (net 15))
 (segment (start 188.402 71.501) (end 188.402 72.705) (width 0.8) (layer F.Cu) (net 15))
 (segment (start 188.402 72.705) (end 188.468 72.771) (width 0.8) (layer F.Cu) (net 15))
 (via (at 188.468 72.771) (size 0.6858) (drill 0.3302) (layers F.Cu B.Cu) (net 15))
 (segment (start 192.659 65.64884) (end 191.389 65.64884) (width 0.8) (layer F.Cu) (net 12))
 (segment (start 193.929 65.64884) (end 192.659 65.64884) (width 0.8) (layer F.Cu) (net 12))
 (segment (start 195.199 65.64884) (end 193.929 65.64884) (width 0.8) (layer F.Cu) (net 12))
 (segment (start 197.739 65.606) (end 195.24184 65.606) (width 0.8) (layer F.Cu) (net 12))
 (segment (start 195.24184 65.606) (end 195.199 65.64884) (width 0.8) (layer F.Cu) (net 12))
 (segment (start 200.40092 65.45326) (end 197.89174 65.45326) (width 0.8) (layer F.Cu) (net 12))
 (segment (start 197.89174 65.45326) (end 197.739 65.606) (width 0.8) (layer F.Cu) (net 12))
 (segment (start 195.199 71.247) (end 195.199 73.72858) (width 0.8) (layer F.Cu) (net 11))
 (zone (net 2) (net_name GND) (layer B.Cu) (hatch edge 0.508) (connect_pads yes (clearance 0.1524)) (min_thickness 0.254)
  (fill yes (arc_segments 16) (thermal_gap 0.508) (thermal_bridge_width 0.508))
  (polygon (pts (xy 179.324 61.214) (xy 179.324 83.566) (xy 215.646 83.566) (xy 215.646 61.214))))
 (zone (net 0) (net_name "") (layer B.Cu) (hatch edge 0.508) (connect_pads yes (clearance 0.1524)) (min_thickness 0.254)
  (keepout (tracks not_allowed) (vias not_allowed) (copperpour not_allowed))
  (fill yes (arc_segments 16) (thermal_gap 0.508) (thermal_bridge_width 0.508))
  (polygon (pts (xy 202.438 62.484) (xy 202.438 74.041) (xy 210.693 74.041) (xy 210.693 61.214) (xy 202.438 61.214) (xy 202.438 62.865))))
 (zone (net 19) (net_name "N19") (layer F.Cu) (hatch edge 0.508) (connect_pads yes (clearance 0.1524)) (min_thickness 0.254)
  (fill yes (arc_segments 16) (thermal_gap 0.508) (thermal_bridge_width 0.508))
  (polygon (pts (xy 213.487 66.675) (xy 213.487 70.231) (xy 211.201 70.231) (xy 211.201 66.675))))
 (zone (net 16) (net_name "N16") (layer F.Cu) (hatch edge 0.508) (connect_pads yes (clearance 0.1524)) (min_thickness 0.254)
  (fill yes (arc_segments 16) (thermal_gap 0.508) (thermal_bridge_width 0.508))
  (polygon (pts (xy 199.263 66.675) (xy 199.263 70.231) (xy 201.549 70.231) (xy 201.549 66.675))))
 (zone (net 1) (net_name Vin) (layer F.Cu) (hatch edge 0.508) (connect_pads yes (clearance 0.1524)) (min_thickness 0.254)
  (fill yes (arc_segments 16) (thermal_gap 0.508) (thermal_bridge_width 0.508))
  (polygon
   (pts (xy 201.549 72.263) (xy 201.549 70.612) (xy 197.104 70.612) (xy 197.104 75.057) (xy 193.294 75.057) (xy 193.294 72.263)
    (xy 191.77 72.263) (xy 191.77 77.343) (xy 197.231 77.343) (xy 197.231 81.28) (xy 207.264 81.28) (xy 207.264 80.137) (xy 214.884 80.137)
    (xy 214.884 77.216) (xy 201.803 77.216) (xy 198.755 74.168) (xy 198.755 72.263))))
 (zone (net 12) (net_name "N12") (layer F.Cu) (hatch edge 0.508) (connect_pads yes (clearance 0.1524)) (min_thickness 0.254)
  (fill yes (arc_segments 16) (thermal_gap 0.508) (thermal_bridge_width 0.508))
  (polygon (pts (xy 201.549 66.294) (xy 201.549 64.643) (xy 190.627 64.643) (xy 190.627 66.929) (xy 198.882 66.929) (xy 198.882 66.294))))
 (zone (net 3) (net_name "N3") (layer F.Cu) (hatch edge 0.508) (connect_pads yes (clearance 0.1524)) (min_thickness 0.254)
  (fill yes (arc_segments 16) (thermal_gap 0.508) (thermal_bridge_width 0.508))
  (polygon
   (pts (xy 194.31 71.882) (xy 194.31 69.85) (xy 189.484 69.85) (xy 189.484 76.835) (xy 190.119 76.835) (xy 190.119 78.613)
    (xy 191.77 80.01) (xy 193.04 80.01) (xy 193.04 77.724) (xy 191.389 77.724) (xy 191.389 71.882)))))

